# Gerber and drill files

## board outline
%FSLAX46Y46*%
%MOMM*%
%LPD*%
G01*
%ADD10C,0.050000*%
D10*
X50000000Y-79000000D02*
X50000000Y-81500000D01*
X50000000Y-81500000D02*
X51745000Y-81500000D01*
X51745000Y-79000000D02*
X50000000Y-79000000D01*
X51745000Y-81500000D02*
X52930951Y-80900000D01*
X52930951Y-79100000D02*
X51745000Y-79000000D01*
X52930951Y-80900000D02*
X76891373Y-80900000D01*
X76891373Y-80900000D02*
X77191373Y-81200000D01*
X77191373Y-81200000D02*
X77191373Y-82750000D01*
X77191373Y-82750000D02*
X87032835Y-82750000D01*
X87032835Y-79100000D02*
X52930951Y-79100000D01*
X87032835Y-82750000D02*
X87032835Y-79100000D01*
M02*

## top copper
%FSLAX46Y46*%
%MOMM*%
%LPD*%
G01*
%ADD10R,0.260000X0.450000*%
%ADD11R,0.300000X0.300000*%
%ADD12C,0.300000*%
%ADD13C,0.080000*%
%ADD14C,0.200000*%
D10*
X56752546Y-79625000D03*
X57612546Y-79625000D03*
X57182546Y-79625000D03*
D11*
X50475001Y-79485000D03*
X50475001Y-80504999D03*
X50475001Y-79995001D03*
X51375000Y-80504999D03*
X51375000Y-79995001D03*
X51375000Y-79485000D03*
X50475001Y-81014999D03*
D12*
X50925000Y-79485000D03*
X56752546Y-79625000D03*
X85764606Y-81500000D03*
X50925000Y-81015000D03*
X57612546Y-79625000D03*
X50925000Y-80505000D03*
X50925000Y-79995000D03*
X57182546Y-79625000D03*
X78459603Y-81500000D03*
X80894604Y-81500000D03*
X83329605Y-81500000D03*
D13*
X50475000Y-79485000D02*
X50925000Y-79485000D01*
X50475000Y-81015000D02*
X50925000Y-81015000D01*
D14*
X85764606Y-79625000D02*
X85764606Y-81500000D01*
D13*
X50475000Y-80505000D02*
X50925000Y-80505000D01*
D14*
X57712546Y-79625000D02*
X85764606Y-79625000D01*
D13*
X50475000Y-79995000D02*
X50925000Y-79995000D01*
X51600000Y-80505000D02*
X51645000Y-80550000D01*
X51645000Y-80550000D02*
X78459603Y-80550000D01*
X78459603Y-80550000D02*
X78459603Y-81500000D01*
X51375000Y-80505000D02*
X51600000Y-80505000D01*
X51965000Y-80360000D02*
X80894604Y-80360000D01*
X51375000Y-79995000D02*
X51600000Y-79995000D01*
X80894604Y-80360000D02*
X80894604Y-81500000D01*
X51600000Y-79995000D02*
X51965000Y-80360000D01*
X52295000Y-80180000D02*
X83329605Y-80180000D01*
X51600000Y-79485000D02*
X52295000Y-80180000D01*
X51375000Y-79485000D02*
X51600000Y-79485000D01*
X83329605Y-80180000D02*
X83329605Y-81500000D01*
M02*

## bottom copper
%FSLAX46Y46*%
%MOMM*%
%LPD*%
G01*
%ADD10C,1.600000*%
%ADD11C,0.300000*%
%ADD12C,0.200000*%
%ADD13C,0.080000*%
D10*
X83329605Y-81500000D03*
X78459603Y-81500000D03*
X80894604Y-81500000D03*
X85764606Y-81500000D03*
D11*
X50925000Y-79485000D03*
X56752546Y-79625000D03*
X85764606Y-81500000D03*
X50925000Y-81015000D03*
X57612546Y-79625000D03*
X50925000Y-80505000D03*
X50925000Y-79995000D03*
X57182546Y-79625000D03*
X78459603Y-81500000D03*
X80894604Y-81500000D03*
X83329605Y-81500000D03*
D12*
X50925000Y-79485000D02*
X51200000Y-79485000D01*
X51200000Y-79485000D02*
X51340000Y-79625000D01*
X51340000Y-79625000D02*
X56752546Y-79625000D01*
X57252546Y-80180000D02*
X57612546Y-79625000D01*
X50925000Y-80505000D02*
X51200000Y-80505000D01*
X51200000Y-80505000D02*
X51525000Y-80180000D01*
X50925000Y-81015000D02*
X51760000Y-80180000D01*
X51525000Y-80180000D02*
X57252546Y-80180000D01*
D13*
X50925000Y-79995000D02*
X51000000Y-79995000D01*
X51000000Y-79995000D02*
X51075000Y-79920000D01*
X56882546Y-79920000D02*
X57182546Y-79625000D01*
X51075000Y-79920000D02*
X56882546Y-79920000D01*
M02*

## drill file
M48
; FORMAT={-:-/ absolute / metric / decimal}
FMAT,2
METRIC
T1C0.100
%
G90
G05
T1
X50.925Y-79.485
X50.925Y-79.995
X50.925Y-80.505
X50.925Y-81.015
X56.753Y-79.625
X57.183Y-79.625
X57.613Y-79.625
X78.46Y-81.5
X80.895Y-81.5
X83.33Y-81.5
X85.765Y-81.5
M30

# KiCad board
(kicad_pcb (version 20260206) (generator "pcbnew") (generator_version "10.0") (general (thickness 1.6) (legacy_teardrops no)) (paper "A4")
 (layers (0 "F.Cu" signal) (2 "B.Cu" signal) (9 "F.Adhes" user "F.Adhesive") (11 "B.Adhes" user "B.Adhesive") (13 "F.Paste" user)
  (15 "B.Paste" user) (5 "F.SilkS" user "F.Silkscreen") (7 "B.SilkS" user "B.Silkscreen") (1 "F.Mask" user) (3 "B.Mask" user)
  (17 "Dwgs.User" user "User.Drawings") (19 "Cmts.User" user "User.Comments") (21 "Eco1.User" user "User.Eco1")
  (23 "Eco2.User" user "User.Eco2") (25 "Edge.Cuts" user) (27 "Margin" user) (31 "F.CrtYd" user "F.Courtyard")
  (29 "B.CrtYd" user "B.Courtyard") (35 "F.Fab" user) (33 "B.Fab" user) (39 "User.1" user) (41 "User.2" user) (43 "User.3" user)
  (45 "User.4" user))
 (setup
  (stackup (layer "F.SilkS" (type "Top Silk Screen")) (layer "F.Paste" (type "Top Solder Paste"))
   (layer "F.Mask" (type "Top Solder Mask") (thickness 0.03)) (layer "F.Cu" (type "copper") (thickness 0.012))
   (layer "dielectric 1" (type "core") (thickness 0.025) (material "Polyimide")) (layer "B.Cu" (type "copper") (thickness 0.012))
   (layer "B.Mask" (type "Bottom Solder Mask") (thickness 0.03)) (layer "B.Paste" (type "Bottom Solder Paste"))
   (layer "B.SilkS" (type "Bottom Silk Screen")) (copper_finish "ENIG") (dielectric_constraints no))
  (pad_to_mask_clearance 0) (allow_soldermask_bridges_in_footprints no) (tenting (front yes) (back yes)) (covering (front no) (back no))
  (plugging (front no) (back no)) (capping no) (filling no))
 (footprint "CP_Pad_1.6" (layer "F.Cu") (at 80.894604 81.5)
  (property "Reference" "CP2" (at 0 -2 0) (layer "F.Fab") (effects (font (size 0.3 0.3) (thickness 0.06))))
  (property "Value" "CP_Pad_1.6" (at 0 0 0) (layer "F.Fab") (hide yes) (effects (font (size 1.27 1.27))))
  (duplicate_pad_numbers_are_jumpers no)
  (pad "1" smd circle (at 0 0) (size 1.6 1.6) (layers "B.Cu" "B.Mask") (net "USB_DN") (solder_mask_margin 0.1)))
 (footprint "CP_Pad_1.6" (layer "F.Cu") (at 85.764606 81.5)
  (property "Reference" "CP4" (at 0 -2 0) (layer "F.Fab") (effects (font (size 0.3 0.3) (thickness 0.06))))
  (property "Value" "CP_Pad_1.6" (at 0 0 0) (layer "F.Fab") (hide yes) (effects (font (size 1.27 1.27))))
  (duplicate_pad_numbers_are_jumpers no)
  (pad "1" smd circle (at 0 0) (size 1.6 1.6) (layers "B.Cu" "B.Mask") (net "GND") (solder_mask_margin 0.1)))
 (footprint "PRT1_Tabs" (layer "F.Cu") (at 57.182546 79.625)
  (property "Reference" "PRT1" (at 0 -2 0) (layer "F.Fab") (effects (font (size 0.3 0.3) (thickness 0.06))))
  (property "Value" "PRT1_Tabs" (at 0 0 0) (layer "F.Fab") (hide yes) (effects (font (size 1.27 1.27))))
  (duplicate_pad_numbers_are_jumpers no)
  (pad "1" smd rect (at -0.43 0) (size 0.26 0.45) (layers "F.Cu" "F.Mask") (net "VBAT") (solder_mask_margin 0.05) (thermal_bridge_angle 45))
  (pad "2" smd rect (at 0.43 0) (size 0.26 0.45) (layers "F.Cu" "F.Mask") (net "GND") (solder_mask_margin 0.05) (thermal_bridge_angle 45))
  (pad "3" smd rect (at 0 0) (size 0.26 0.45) (layers "F.Cu" "F.Mask") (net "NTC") (solder_mask_margin 0.05) (thermal_bridge_angle 45)))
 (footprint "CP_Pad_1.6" (layer "F.Cu") (at 83.329605 81.5)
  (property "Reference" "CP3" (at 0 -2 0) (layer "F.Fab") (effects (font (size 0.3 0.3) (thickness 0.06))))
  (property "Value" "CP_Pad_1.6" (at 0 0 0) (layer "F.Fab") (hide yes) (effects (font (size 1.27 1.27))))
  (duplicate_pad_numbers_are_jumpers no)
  (pad "1" smd circle (at 0 0) (size 1.6 1.6) (layers "B.Cu" "B.Mask") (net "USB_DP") (solder_mask_margin 0.1)))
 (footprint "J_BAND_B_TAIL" (layer "F.Cu") (at 50.9 80.25)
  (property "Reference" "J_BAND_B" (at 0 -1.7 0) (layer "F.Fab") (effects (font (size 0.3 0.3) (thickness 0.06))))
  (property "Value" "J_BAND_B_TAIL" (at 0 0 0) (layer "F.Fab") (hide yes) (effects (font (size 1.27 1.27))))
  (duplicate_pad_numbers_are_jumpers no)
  (pad "1" smd rect (at -0.424999 -0.765) (size 0.3 0.3) (layers "F.Cu" "F.Mask") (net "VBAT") (solder_mask_margin 0.05)
   (thermal_bridge_angle 45))
  (pad "2" smd rect (at -0.424999 0.254999) (size 0.3 0.3) (layers "F.Cu" "F.Mask") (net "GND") (solder_mask_margin 0.05)
   (thermal_bridge_angle 45))
  (pad "3" smd rect (at -0.424999 -0.254999) (size 0.3 0.3) (layers "F.Cu" "F.Mask") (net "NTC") (solder_mask_margin 0.05)
   (thermal_bridge_angle 45))
  (pad "4" smd rect (at 0.475 0.254999) (size 0.3 0.3) (layers "F.Cu" "F.Mask") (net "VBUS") (solder_mask_margin 0.05)
   (thermal_bridge_angle 45))
  (pad "5" smd rect (at 0.475 -0.254999) (size 0.3 0.3) (layers "F.Cu" "F.Mask") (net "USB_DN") (solder_mask_margin 0.05)
   (thermal_bridge_angle 45))
  (pad "6" smd rect (at 0.475 -0.765) (size 0.3 0.3) (layers "F.Cu" "F.Mask") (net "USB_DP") (solder_mask_margin 0.05)
   (thermal_bridge_angle 45))
  (pad "7" smd rect (at -0.424999 0.764999) (size 0.3 0.3) (layers "F.Cu" "F.Mask") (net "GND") (solder_mask_margin 0.05)
   (thermal_bridge_angle 45)))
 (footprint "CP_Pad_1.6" (layer "F.Cu") (at 78.459603 81.5)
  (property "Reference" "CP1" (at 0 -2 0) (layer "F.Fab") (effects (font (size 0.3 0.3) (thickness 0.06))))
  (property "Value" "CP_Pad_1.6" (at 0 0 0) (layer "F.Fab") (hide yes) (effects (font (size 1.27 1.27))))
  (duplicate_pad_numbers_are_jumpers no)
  (pad "1" smd circle (at 0 0) (size 1.6 1.6) (layers "B.Cu" "B.Mask") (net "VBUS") (solder_mask_margin 0.1)))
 (gr_line (start 50 79) (end 50 81.5) (stroke (width 0.05) (type default)) (layer "Edge.Cuts"))
 (gr_line (start 50 81.5) (end 51.745 81.5) (stroke (width 0.05) (type default)) (layer "Edge.Cuts"))
 (gr_line (start 51.745 79) (end 50 79) (stroke (width 0.05) (type default)) (layer "Edge.Cuts"))
 (gr_line (start 51.745 81.5) (end 52.930951 80.9) (stroke (width 0.05) (type default)) (layer "Edge.Cuts"))
 (gr_line (start 52.930951 79.1) (end 51.745 79) (stroke (width 0.05) (type default)) (layer "Edge.Cuts"))
 (gr_line (start 52.930951 80.9) (end 76.891373 80.9) (stroke (width 0.05) (type default)) (layer "Edge.Cuts"))
 (gr_line (start 76.891373 80.9) (end 77.191373 81.2) (stroke (width 0.05) (type default)) (layer "Edge.Cuts"))
 (gr_line (start 77.191373 81.2) (end 77.191373 82.75) (stroke (width 0.05) (type default)) (layer "Edge.Cuts"))
 (gr_line (start 77.191373 82.75) (end 87.032835 82.75) (stroke (width 0.05) (type default)) (layer "Edge.Cuts"))
 (gr_line (start 87.032835 79.1) (end 52.930951 79.1) (stroke (width 0.05) (type default)) (layer "Edge.Cuts"))
 (gr_line (start 87.032835 82.75) (end 87.032835 79.1) (stroke (width 0.05) (type default)) (layer "Edge.Cuts"))
 (segment (start 50.475 79.485) (end 50.925 79.485) (width 0.08) (layer "F.Cu") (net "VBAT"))
 (via (at 56.752546 79.625) (size 0.3) (drill 0.1) (layers "F.Cu" "B.Cu") (tenting (front yes) (back yes)) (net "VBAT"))
 (via (at 50.925 79.485) (size 0.3) (drill 0.1) (layers "F.Cu" "B.Cu") (tenting (front yes) (back yes)) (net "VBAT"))
 (segment (start 50.925 79.485) (end 51.2 79.485) (width 0.2) (layer "B.Cu") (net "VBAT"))
 (segment (start 51.2 79.485) (end 51.34 79.625) (width 0.2) (layer "B.Cu") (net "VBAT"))
 (segment (start 51.34 79.625) (end 56.752546 79.625) (width 0.2) (layer "B.Cu") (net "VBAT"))
 (segment (start 57.712546 79.625) (end 85.764606 79.625) (width 0.2) (layer "F.Cu") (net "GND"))
 (segment (start 50.475 80.505) (end 50.925 80.505) (width 0.08) (layer "F.Cu") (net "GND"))
 (segment (start 50.475 81.015) (end 50.925 81.015) (width 0.08) (layer "F.Cu") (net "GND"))
 (segment (start 85.764606 79.625) (end 85.764606 81.5) (width 0.2) (layer "F.Cu") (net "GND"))
 (via (at 50.925 81.015) (size 0.3) (drill 0.1) (layers "F.Cu" "B.Cu") (tenting (front yes) (back yes)) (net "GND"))
 (via (at 85.764606 81.5) (size 0.3) (drill 0.1) (layers "F.Cu" "B.Cu") (tenting (front yes) (back yes)) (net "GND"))
 (via (at 57.612546 79.625) (size 0.3) (drill 0.1) (layers "F.Cu" "B.Cu") (tenting (front yes) (back yes)) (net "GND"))
 (via (at 50.925 80.505) (size 0.3) (drill 0.1) (layers "F.Cu" "B.Cu") (tenting (front yes) (back yes)) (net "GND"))
 (segment (start 51.2 80.505) (end 51.525 80.18) (width 0.2) (layer "B.Cu") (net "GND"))
 (segment (start 50.925 80.505) (end 51.2 80.505) (width 0.2) (layer "B.Cu") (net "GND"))
 (segment (start 51.525 80.18) (end 57.252546 80.18) (width 0.2) (layer "B.Cu") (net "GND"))
 (segment (start 50.925 81.015) (end 51.76 80.18) (width 0.2) (layer "B.Cu") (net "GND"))
 (segment (start 57.252546 80.18) (end 57.612546 79.625) (width 0.2) (layer "B.Cu") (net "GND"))
 (segment (start 50.475 79.995) (end 50.925 79.995) (width 0.08) (layer "F.Cu") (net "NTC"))
 (via (at 50.925 79.995) (size 0.3) (drill 0.1) (layers "F.Cu" "B.Cu") (tenting (front yes) (back yes)) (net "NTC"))
 (via (at 57.182546 79.625) (size 0.3) (drill 0.1) (layers "F.Cu" "B.Cu") (tenting (front yes) (back yes)) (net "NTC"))
 (segment (start 56.882546 79.92) (end 57.182546 79.625) (width 0.08) (layer "B.Cu") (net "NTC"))
 (segment (start 50.925 79.995) (end 51 79.995) (width 0.08) (layer "B.Cu") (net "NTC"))
 (segment (start 51 79.995) (end 51.075 79.92) (width 0.08) (layer "B.Cu") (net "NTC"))
 (segment (start 51.075 79.92) (end 56.882546 79.92) (width 0.08) (layer "B.Cu") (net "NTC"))
 (segment (start 78.459603 80.55) (end 78.459603 81.5) (width 0.08) (layer "F.Cu") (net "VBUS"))
 (segment (start 51.645 80.55) (end 78.459603 80.55) (width 0.08) (layer "F.Cu") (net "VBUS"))
 (segment (start 51.6 80.505) (end 51.645 80.55) (width 0.08) (layer "F.Cu") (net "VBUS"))
 (segment (start 51.375 80.505) (end 51.6 80.505) (width 0.08) (layer "F.Cu") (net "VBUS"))
 (via (at 78.459603 81.5) (size 0.3) (drill 0.1) (layers "F.Cu" "B.Cu") (tenting (front yes) (back yes)) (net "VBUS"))
 (segment (start 51.965 80.36) (end 80.894604 80.36) (width 0.08) (layer "F.Cu") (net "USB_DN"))
 (segment (start 80.894604 80.36) (end 80.894604 81.5) (width 0.08) (layer "F.Cu") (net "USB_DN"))
 (segment (start 51.6 79.995) (end 51.965 80.36) (width 0.08) (layer "F.Cu") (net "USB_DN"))
 (segment (start 51.375 79.995) (end 51.6 79.995) (width 0.08) (layer "F.Cu") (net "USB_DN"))
 (via (at 80.894604 81.5) (size 0.3) (drill 0.1) (layers "F.Cu" "B.Cu") (tenting (front yes) (back yes)) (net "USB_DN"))
 (segment (start 51.375 79.485) (end 51.6 79.485) (width 0.08) (layer "F.Cu") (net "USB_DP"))
 (segment (start 51.6 79.485) (end 52.295 80.18) (width 0.08) (layer "F.Cu") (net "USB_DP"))
 (segment (start 83.329605 80.18) (end 83.329605 81.5) (width 0.08) (layer "F.Cu") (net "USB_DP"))
 (segment (start 52.295 80.18) (end 83.329605 80.18) (width 0.08) (layer "F.Cu") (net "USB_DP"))
 (via (at 83.329605 81.5) (size 0.3) (drill 0.1) (layers "F.Cu" "B.Cu") (tenting (front yes) (back yes)) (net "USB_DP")))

